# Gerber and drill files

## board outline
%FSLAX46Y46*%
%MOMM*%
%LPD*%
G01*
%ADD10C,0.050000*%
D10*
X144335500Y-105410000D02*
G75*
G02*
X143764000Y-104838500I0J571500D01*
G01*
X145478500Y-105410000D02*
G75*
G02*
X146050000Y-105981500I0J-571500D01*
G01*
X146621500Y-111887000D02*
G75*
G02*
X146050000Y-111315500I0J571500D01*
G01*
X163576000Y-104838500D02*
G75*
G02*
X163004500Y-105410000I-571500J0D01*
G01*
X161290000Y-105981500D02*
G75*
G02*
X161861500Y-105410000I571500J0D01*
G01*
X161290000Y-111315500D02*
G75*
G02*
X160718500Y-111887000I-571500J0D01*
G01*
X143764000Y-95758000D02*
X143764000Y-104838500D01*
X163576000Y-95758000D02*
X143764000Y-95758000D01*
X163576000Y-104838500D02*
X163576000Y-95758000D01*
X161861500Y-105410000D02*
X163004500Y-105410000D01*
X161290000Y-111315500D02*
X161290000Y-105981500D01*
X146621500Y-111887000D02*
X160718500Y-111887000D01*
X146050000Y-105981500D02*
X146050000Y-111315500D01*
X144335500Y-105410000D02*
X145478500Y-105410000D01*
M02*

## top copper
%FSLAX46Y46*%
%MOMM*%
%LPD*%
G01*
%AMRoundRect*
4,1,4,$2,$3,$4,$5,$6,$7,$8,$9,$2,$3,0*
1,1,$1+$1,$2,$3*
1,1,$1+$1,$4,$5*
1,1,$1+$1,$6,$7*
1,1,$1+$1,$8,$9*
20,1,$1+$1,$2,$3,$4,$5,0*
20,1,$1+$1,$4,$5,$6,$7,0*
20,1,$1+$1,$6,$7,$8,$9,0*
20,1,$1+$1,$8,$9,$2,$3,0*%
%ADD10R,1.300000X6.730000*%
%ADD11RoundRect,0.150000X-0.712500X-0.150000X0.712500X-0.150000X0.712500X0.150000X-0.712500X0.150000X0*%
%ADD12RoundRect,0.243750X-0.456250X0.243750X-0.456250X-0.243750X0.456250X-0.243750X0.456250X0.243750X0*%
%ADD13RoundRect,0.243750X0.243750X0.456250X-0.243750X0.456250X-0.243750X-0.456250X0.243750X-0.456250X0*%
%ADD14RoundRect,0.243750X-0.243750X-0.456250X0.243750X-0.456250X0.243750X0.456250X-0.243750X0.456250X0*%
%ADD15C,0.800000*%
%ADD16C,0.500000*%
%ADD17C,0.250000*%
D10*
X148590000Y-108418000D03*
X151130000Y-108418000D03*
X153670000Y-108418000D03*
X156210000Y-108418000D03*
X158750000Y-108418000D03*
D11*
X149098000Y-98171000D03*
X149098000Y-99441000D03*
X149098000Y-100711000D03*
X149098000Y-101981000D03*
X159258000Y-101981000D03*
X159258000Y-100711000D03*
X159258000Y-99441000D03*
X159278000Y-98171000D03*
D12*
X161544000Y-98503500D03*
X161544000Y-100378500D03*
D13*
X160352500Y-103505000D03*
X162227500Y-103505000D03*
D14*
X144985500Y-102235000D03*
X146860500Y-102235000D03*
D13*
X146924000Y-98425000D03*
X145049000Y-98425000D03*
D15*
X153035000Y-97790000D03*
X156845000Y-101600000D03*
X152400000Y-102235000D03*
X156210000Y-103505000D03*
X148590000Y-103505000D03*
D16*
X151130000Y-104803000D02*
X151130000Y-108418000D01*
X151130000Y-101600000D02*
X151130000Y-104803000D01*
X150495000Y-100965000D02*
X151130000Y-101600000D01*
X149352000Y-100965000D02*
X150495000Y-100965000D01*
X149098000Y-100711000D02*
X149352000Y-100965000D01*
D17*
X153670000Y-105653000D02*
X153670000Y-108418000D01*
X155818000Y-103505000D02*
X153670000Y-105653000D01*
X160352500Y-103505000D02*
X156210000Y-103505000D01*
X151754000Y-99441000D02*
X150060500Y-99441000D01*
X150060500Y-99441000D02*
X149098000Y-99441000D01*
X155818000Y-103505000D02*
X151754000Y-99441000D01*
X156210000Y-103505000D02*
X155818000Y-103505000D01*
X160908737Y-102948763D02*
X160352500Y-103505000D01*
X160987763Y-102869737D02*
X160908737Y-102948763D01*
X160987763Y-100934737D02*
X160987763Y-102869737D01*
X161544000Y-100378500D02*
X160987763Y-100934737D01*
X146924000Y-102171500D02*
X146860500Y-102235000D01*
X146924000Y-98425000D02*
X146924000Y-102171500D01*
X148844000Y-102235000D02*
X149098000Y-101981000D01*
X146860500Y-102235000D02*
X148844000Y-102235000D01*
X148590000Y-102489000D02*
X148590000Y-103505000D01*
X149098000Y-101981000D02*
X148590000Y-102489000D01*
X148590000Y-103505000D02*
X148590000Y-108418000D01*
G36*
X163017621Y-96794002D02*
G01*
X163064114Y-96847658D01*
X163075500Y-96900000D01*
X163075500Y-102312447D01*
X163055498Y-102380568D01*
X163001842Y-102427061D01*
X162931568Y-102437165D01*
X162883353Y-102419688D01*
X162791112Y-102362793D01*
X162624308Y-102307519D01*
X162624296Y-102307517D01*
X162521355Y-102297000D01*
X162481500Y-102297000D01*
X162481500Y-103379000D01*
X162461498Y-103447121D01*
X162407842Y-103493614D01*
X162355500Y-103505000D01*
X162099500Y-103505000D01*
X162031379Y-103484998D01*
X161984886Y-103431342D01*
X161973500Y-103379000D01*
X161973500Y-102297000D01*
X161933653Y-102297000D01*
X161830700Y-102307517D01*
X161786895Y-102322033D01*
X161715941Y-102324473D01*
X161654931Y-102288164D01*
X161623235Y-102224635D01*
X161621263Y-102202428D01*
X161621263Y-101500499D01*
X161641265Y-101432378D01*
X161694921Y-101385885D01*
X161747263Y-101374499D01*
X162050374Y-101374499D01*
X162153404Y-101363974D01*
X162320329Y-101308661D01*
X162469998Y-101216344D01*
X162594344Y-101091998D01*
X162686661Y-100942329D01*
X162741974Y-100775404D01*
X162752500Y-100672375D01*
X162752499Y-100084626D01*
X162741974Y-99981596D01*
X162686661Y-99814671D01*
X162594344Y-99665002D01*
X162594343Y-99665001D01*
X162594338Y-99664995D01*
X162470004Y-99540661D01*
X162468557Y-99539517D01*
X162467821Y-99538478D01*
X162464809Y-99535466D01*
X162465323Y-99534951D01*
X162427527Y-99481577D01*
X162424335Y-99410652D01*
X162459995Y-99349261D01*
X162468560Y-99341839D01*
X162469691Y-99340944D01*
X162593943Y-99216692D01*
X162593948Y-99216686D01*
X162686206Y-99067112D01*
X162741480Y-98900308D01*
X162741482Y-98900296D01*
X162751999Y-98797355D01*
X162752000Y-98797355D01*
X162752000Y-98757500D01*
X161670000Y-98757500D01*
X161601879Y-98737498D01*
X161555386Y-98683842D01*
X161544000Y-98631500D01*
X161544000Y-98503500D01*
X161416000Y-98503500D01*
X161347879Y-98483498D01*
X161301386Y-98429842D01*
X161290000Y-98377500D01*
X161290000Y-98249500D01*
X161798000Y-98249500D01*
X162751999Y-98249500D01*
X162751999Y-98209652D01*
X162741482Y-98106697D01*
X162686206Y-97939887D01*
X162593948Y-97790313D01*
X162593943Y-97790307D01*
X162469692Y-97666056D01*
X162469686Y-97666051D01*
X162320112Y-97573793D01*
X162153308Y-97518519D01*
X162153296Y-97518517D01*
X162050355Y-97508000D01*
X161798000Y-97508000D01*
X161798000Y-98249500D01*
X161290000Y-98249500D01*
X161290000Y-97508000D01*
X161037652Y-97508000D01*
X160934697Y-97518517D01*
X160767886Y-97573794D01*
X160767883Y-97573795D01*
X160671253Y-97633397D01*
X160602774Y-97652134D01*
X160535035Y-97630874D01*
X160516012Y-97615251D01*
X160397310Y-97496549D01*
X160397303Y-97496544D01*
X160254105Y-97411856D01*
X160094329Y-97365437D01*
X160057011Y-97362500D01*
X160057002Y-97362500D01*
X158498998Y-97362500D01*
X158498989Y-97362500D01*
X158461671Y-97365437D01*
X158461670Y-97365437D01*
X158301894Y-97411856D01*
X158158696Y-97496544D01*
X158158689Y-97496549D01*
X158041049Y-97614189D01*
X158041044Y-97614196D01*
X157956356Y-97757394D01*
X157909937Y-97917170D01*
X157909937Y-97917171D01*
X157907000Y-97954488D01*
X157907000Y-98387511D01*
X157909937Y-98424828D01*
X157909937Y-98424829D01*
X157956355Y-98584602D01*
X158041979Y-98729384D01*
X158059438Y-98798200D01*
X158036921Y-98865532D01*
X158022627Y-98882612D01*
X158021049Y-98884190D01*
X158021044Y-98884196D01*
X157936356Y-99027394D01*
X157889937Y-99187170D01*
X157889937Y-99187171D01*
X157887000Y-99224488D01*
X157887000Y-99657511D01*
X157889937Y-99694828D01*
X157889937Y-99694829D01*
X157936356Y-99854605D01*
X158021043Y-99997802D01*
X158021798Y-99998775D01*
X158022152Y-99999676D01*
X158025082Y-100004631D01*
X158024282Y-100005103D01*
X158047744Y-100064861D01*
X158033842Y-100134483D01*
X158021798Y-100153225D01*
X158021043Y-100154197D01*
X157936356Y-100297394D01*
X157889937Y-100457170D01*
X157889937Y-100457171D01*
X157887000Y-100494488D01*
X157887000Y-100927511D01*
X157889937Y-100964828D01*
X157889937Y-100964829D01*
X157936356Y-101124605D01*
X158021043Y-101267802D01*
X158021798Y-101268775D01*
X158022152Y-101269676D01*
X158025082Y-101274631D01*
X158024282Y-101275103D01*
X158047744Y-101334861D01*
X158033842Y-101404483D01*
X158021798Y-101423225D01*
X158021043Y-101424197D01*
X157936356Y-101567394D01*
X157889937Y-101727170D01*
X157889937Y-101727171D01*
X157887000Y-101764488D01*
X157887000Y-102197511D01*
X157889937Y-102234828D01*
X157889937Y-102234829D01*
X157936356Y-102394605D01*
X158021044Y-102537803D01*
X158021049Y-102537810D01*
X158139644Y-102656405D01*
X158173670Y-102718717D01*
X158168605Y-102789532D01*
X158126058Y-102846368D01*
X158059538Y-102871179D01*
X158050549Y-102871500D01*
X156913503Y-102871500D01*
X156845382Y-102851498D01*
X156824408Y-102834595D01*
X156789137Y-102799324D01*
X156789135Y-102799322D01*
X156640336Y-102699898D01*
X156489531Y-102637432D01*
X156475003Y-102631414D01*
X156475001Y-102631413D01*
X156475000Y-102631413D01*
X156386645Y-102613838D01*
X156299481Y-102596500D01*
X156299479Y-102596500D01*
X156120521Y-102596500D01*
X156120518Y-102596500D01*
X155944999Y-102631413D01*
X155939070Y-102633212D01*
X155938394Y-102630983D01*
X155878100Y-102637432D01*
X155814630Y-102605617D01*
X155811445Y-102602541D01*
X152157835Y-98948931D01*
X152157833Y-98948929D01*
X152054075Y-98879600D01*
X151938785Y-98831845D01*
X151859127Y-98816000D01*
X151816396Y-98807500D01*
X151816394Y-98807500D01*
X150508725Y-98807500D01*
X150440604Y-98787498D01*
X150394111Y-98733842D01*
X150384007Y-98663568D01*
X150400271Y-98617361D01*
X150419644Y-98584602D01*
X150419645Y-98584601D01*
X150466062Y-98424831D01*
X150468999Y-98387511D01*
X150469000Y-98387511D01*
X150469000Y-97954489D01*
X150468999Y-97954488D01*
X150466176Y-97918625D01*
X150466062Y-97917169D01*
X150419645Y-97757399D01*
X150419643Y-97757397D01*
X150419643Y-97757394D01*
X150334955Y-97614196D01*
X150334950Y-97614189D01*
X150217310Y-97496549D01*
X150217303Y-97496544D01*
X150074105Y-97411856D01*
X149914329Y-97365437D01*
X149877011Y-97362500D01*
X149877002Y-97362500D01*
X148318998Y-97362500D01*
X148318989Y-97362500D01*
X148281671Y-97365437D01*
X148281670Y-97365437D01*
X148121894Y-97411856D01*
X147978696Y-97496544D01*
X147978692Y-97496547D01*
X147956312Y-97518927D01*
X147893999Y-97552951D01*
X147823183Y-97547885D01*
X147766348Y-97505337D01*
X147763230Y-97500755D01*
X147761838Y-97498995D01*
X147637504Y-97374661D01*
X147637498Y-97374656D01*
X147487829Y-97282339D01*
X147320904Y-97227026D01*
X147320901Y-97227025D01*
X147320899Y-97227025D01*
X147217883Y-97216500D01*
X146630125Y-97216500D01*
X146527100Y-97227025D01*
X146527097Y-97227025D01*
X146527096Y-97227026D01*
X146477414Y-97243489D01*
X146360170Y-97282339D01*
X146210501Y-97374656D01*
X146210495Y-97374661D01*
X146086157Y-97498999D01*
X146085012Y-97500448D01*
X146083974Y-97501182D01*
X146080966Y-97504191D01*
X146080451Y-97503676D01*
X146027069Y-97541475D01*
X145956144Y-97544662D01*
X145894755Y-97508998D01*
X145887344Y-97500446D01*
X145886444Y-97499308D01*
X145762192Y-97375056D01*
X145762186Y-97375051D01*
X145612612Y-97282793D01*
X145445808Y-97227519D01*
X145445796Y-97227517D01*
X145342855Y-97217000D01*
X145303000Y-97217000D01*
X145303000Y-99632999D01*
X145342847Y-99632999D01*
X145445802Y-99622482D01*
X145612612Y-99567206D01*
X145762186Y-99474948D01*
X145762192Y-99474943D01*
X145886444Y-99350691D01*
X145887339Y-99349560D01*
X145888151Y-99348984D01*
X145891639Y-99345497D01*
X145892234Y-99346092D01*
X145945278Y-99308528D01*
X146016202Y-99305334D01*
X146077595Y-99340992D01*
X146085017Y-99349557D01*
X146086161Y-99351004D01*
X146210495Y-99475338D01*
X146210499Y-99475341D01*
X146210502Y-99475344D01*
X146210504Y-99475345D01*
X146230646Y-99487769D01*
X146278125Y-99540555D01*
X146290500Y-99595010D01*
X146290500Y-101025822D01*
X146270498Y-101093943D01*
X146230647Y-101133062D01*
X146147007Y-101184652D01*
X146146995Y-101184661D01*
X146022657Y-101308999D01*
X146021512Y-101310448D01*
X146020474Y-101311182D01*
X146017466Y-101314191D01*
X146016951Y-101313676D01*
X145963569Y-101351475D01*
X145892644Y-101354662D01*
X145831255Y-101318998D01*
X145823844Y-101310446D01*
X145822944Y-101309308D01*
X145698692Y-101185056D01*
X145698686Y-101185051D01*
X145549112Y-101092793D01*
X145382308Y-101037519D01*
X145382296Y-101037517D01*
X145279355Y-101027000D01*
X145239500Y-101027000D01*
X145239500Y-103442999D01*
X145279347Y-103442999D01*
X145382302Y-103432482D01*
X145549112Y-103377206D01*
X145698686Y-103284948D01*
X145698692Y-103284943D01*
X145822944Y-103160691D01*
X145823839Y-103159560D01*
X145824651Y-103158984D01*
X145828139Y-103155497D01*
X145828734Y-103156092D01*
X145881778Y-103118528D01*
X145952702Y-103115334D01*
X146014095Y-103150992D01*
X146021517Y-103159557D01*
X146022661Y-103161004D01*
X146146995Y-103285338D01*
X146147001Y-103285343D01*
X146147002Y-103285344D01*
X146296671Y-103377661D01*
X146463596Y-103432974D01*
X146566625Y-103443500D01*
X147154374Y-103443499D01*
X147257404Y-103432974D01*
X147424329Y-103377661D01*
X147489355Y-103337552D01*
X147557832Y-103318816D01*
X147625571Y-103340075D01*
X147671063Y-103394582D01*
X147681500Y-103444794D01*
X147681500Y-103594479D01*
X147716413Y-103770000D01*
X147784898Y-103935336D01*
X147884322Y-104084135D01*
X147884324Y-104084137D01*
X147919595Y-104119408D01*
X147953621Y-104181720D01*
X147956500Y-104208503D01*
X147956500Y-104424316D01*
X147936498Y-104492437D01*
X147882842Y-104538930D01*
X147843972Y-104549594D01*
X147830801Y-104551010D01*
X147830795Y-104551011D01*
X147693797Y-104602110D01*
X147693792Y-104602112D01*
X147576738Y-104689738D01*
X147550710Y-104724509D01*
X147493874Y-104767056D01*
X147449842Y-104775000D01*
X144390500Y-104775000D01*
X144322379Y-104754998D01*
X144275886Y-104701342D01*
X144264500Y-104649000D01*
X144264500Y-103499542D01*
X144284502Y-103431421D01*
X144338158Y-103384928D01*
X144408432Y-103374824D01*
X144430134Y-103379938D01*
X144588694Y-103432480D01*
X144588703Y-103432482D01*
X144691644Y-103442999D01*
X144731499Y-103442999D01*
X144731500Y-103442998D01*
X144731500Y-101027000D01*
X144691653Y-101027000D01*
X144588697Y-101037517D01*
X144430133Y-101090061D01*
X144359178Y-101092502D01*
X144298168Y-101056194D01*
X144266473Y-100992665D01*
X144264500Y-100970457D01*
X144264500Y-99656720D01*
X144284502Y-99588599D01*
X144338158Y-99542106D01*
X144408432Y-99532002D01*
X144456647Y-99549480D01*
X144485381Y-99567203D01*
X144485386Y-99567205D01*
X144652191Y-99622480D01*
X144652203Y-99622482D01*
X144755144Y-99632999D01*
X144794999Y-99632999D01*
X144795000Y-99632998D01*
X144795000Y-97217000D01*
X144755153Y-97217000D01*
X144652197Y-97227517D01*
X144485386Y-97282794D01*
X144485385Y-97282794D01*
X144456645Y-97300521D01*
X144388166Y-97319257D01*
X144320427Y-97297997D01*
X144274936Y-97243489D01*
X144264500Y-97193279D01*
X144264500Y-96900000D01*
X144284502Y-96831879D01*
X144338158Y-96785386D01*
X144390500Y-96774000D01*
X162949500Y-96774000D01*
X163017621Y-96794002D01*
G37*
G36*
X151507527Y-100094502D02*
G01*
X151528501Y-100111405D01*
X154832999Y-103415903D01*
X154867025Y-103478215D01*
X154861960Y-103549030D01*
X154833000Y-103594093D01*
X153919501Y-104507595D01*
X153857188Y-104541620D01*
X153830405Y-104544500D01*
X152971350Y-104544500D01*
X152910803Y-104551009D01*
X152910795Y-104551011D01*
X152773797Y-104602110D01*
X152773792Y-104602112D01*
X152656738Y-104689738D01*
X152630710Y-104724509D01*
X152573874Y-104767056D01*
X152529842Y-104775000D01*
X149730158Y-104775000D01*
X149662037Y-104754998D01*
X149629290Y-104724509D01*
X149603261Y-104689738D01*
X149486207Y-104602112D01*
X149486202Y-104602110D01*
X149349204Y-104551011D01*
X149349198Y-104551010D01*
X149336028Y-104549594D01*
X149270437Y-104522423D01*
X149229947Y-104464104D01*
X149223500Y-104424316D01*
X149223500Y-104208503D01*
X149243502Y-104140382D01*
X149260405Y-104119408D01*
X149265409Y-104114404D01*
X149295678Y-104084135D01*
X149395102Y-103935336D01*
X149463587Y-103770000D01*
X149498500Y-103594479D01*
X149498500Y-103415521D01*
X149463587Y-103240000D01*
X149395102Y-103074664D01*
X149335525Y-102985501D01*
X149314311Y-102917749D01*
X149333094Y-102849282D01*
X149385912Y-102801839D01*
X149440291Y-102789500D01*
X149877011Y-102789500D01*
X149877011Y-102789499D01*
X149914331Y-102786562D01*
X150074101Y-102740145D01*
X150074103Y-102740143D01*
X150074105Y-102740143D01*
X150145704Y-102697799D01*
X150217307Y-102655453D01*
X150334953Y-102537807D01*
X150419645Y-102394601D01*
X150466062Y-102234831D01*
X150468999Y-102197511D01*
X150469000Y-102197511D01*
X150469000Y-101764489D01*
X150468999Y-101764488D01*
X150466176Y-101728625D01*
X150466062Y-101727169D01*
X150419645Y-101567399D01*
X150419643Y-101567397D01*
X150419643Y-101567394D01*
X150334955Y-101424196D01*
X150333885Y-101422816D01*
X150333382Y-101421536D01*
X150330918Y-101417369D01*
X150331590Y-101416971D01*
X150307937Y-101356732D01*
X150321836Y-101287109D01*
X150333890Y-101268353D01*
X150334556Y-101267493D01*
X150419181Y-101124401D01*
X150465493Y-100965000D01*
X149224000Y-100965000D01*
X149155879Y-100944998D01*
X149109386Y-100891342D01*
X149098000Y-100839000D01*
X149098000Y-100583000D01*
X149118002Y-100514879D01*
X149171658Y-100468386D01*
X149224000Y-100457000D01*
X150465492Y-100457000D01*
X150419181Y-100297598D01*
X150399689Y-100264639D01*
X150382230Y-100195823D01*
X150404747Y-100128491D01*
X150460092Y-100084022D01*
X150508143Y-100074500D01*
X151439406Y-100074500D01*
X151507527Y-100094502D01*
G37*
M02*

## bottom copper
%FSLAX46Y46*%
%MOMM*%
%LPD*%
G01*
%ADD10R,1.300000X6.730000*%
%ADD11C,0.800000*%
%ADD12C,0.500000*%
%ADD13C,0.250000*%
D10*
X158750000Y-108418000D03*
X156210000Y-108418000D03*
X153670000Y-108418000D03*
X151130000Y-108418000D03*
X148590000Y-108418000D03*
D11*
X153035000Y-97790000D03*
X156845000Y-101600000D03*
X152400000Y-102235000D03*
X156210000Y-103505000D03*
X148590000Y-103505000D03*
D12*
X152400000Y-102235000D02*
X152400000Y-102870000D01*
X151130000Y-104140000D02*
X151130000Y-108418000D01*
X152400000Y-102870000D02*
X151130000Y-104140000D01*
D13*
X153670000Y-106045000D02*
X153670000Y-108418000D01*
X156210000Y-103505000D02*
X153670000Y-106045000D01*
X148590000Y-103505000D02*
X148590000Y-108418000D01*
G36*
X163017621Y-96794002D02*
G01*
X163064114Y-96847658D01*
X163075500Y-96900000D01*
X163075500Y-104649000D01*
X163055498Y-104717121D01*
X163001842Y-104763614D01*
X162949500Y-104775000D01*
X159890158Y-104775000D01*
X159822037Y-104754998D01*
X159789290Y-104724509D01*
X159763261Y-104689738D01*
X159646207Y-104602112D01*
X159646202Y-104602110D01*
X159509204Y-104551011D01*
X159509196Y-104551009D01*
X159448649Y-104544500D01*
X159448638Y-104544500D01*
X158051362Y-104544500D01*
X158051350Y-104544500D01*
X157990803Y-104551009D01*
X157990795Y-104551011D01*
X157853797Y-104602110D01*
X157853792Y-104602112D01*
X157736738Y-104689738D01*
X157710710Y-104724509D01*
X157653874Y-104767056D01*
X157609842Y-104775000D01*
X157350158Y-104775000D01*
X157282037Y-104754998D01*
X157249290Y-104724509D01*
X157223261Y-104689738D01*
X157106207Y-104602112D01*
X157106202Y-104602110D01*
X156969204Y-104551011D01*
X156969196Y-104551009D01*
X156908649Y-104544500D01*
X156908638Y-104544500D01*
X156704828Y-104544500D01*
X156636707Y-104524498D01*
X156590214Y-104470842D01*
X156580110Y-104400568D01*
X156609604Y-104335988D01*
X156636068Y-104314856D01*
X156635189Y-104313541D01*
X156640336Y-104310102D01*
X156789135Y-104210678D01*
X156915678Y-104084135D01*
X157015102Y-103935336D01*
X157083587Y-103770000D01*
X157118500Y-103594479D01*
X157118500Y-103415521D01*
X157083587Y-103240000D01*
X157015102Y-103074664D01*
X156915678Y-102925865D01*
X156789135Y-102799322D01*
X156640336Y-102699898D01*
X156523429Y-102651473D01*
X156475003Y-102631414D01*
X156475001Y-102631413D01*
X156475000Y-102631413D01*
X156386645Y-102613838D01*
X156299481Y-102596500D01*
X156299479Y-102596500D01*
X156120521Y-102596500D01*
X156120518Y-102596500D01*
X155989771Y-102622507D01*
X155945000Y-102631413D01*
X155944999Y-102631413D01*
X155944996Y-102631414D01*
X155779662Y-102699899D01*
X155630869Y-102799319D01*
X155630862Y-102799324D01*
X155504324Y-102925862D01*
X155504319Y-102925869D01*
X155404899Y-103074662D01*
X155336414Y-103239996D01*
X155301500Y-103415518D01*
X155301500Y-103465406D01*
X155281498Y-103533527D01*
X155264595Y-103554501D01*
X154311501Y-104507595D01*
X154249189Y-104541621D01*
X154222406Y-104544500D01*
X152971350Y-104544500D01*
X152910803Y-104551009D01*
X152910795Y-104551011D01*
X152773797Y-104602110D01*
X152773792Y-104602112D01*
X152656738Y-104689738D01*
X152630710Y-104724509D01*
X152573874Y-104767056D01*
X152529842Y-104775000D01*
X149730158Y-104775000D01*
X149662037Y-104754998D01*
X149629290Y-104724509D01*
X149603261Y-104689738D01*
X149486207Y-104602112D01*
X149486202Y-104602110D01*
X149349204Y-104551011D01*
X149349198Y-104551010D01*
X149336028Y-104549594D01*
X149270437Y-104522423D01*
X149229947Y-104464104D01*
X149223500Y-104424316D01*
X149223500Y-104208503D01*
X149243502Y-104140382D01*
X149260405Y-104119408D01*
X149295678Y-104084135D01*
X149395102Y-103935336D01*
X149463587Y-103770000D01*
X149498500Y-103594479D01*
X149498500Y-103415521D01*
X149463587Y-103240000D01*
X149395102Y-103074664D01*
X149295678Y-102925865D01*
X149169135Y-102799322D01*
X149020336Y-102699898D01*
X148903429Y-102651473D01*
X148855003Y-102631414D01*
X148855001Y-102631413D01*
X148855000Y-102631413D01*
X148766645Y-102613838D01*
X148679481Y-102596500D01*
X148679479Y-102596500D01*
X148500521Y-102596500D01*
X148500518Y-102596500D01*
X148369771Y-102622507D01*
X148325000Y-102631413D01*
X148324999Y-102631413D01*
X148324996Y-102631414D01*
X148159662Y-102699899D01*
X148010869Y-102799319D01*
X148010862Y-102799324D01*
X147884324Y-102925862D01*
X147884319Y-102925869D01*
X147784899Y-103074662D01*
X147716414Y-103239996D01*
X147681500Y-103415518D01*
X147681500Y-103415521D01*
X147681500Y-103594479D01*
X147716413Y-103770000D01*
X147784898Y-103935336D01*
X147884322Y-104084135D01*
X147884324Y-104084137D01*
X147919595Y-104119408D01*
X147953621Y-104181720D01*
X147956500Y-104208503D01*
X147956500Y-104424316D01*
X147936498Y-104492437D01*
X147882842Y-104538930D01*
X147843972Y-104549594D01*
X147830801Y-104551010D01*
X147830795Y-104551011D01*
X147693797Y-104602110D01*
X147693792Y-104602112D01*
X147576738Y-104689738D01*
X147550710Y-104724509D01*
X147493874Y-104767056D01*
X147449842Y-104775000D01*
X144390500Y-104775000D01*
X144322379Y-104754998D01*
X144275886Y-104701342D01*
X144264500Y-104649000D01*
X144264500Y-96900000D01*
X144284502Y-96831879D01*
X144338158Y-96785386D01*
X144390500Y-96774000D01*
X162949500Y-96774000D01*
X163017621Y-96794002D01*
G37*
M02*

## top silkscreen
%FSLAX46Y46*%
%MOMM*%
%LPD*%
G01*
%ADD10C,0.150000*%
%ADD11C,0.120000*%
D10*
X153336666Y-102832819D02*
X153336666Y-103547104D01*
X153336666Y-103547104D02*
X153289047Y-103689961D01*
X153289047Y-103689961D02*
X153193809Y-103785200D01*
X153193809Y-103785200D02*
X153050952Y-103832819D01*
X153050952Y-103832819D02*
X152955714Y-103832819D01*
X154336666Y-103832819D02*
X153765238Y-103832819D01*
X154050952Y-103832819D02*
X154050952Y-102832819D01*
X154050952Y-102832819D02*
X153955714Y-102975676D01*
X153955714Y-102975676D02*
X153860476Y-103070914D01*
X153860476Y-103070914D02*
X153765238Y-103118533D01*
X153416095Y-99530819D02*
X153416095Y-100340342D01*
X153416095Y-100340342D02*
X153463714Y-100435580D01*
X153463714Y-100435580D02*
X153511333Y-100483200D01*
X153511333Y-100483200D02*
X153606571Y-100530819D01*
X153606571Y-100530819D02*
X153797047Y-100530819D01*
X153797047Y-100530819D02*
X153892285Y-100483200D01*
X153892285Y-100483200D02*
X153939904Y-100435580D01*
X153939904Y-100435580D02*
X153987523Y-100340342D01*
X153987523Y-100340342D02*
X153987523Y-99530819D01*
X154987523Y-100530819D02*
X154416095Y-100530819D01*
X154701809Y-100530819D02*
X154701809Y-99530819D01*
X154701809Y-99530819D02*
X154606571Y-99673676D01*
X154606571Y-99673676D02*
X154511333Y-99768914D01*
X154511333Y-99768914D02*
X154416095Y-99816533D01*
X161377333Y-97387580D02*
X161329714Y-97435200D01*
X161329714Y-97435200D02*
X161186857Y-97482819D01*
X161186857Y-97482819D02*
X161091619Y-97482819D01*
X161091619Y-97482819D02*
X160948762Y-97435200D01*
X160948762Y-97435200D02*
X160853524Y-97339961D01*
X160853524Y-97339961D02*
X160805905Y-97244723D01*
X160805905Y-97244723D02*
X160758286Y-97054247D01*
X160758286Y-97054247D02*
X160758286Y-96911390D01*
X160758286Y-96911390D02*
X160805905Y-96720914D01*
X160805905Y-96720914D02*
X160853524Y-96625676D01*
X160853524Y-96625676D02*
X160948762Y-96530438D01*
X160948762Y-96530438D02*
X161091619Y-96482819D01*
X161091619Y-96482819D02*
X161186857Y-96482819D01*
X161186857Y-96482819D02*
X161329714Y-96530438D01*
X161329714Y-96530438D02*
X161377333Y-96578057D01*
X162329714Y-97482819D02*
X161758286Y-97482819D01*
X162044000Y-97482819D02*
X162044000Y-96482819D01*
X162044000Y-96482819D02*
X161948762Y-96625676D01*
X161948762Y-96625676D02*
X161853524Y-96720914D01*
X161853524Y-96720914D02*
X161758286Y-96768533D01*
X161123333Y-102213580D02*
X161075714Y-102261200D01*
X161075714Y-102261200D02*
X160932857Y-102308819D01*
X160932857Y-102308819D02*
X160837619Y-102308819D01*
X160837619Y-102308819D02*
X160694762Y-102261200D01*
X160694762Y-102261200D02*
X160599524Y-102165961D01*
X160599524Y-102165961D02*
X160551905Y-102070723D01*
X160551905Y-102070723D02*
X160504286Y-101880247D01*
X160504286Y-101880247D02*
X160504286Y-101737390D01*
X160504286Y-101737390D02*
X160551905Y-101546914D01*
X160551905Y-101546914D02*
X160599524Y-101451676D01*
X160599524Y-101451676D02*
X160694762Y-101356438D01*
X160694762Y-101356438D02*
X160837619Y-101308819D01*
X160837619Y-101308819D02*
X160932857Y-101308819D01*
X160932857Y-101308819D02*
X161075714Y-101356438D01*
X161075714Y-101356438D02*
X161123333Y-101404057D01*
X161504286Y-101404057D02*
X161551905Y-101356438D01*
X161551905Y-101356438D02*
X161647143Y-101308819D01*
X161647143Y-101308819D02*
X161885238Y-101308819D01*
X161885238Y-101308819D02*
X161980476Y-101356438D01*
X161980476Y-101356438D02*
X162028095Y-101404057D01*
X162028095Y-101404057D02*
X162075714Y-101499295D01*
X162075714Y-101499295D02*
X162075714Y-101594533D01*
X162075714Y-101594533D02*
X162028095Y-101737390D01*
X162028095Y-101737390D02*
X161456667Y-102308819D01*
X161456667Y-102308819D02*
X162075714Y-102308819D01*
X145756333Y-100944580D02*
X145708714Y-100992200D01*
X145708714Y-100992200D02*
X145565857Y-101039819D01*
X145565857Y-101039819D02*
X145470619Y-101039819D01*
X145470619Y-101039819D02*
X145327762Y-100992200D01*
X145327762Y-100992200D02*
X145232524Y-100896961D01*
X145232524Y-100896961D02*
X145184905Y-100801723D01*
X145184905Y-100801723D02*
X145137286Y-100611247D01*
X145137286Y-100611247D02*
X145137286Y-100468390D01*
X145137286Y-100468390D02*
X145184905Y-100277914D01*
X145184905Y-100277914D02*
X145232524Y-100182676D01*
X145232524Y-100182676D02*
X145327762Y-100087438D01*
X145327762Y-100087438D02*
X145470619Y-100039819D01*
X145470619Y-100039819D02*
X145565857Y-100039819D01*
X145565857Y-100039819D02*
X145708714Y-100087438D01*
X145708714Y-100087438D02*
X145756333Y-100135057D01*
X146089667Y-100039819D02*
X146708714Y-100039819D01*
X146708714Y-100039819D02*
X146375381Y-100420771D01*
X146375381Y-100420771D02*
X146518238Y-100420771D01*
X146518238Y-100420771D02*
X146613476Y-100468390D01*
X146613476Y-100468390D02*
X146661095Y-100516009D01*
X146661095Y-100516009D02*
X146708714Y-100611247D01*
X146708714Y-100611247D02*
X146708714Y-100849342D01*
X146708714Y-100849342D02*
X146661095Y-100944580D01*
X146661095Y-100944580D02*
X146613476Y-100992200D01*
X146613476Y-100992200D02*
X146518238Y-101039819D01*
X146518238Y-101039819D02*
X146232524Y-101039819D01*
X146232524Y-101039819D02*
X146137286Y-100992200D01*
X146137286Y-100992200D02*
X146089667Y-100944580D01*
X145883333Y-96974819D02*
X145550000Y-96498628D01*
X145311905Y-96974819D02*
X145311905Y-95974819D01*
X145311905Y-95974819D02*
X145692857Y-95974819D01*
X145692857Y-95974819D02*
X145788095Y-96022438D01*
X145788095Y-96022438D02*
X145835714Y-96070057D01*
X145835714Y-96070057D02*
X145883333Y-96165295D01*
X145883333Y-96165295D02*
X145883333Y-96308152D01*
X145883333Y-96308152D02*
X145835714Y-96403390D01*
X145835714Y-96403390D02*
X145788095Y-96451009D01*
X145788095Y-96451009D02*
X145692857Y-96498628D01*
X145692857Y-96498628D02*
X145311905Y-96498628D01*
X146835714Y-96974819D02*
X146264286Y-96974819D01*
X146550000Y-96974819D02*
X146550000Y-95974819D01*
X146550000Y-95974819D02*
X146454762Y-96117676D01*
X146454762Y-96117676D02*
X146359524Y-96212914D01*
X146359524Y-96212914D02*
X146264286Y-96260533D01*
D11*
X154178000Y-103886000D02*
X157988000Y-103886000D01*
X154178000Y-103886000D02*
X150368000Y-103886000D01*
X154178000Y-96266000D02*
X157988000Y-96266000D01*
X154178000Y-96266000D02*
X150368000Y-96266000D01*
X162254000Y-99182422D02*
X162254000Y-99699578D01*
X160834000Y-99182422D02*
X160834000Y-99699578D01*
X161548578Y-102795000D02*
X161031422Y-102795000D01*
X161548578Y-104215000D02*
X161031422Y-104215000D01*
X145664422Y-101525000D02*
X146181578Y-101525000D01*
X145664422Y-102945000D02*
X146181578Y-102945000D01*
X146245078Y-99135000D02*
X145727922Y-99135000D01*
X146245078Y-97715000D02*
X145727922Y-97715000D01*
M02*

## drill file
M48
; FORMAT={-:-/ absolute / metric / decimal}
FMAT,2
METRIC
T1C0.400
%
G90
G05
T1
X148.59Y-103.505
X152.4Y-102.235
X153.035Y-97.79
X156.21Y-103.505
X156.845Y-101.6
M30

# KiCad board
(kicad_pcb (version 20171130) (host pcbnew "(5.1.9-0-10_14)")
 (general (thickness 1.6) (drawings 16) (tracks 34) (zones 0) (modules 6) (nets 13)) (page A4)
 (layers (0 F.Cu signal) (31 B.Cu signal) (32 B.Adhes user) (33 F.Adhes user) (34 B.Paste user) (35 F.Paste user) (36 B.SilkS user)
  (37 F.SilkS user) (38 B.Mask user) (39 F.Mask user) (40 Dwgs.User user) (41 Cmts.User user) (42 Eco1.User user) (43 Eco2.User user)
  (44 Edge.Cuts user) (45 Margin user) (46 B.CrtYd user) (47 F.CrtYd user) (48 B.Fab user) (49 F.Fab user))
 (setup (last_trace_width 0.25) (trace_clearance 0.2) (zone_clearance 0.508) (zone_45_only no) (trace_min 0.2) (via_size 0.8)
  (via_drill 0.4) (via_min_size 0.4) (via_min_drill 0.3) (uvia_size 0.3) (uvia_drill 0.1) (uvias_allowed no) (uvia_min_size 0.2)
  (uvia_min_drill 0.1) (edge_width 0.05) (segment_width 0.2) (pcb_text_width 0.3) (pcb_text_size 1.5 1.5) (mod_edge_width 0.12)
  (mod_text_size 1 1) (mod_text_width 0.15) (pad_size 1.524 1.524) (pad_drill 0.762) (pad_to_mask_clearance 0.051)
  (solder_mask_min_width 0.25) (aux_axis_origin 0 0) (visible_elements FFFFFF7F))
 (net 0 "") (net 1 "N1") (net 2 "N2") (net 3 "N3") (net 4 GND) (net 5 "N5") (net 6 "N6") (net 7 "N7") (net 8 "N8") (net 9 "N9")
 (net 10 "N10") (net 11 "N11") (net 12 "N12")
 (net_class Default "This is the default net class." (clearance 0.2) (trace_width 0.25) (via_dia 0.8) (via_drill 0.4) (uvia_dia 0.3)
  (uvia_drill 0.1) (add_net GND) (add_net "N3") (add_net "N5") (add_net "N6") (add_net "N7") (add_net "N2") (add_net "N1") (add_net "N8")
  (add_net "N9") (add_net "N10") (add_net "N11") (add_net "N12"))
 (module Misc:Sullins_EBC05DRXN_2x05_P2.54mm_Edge (layer F.Cu) (at 148.59 105.918)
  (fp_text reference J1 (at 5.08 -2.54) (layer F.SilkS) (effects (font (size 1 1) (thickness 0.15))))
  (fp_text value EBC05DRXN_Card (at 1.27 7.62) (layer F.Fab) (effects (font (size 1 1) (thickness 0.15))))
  (pad B5 connect rect (at 10.16 2.5) (size 1.3 6.73) (layers B.Cu) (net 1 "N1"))
  (pad B4 connect rect (at 7.62 2.5) (size 1.3 6.73) (layers B.Cu) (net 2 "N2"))
  (pad B3 connect rect (at 5.08 2.5) (size 1.3 6.73) (layers B.Cu) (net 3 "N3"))
  (pad B2 connect rect (at 2.54 2.5) (size 1.3 6.73) (layers B.Cu) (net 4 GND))
  (pad B1 connect rect (at 0 2.5) (size 1.3 6.73) (layers B.Cu) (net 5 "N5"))
  (pad A1 connect rect (at 0 2.5) (size 1.3 6.73) (layers F.Cu) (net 5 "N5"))
  (pad A2 connect rect (at 2.54 2.5) (size 1.3 6.73) (layers F.Cu) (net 4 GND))
  (pad A3 connect rect (at 5.08 2.5) (size 1.3 6.73) (layers F.Cu) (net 3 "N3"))
  (pad A4 connect rect (at 7.62 2.5) (size 1.3 6.73) (layers F.Cu) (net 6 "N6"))
  (pad A5 connect rect (at 10.16 2.5) (size 1.3 6.73) (layers F.Cu) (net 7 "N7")))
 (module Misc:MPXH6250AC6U (layer F.Cu) (at 154.178 100.076)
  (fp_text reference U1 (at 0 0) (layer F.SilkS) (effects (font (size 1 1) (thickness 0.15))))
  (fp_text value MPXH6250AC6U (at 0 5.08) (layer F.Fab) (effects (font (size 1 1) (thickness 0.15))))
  (fp_line (start 0 3.81) (end 3.81 3.81) (layer F.SilkS) (width 0.12))
  (fp_line (start 0 3.81) (end -3.81 3.81) (layer F.SilkS) (width 0.12))
  (fp_line (start 0 -3.81) (end 3.81 -3.81) (layer F.SilkS) (width 0.12))
  (fp_line (start 0 -3.81) (end -3.81 -3.81) (layer F.SilkS) (width 0.12))
  (pad 1 smd roundrect (at -5.08 -1.905) (size 1.725 0.6) (layers F.Cu F.Paste F.Mask) (roundrect_rratio 0.25) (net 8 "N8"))
  (pad 2 smd roundrect (at -5.08 -0.635) (size 1.725 0.6) (layers F.Cu F.Paste F.Mask) (roundrect_rratio 0.25) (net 3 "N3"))
  (pad 3 smd roundrect (at -5.08 0.635) (size 1.725 0.6) (layers F.Cu F.Paste F.Mask) (roundrect_rratio 0.25) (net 4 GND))
  (pad 4 smd roundrect (at -5.08 1.905) (size 1.725 0.6) (layers F.Cu F.Paste F.Mask) (roundrect_rratio 0.25) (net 5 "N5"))
  (pad 5 smd roundrect (at 5.08 1.905) (size 1.725 0.6) (layers F.Cu F.Paste F.Mask) (roundrect_rratio 0.25) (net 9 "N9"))
  (pad 6 smd roundrect (at 5.08 0.635) (size 1.725 0.6) (layers F.Cu F.Paste F.Mask) (roundrect_rratio 0.25) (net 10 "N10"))
  (pad 7 smd roundrect (at 5.08 -0.635) (size 1.725 0.6) (layers F.Cu F.Paste F.Mask) (roundrect_rratio 0.25) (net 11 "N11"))
  (pad 8 smd roundrect (at 5.1 -1.905) (size 1.725 0.6) (layers F.Cu F.Paste F.Mask) (roundrect_rratio 0.25) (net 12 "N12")))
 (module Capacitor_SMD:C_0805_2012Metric (layer F.Cu) (at 161.544 99.441 270)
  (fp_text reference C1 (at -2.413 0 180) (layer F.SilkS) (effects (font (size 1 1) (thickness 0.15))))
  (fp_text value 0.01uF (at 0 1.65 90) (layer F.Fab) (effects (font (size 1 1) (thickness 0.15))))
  (fp_line (start -0.258578 -0.71) (end 0.258578 -0.71) (layer F.SilkS) (width 0.12))
  (fp_line (start -0.258578 0.71) (end 0.258578 0.71) (layer F.SilkS) (width 0.12))
  (pad 1 smd roundrect (at -0.9375 0 270) (size 0.975 1.4) (layers F.Cu F.Paste F.Mask) (roundrect_rratio 0.25) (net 4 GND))
  (pad 2 smd roundrect (at 0.9375 0 270) (size 0.975 1.4) (layers F.Cu F.Paste F.Mask) (roundrect_rratio 0.25) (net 3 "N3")))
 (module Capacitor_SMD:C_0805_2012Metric (layer F.Cu) (at 161.29 103.505 180)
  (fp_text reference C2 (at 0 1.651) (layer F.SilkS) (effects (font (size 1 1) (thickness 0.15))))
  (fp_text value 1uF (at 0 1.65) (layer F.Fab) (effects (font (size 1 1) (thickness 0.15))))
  (fp_line (start -0.258578 0.71) (end 0.258578 0.71) (layer F.SilkS) (width 0.12))
  (fp_line (start -0.258578 -0.71) (end 0.258578 -0.71) (layer F.SilkS) (width 0.12))
  (pad 2 smd roundrect (at 0.9375 0 180) (size 0.975 1.4) (layers F.Cu F.Paste F.Mask) (roundrect_rratio 0.25) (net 3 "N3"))
  (pad 1 smd roundrect (at -0.9375 0 180) (size 0.975 1.4) (layers F.Cu F.Paste F.Mask) (roundrect_rratio 0.25) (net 4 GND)))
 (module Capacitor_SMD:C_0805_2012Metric (layer F.Cu) (at 145.923 102.235)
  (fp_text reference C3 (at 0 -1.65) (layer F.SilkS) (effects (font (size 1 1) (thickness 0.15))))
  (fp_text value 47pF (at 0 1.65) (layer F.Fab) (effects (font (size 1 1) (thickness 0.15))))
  (fp_line (start -0.258578 -0.71) (end 0.258578 -0.71) (layer F.SilkS) (width 0.12))
  (fp_line (start -0.258578 0.71) (end 0.258578 0.71) (layer F.SilkS) (width 0.12))
  (pad 1 smd roundrect (at -0.9375 0) (size 0.975 1.4) (layers F.Cu F.Paste F.Mask) (roundrect_rratio 0.25) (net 4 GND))
  (pad 2 smd roundrect (at 0.9375 0) (size 0.975 1.4) (layers F.Cu F.Paste F.Mask) (roundrect_rratio 0.25) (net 5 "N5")))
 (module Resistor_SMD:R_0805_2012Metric (layer F.Cu) (at 145.9865 98.425 180)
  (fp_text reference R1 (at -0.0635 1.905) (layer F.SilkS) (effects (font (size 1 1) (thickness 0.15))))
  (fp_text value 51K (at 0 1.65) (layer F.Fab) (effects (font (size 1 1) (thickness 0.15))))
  (fp_line (start -0.258578 -0.71) (end 0.258578 -0.71) (layer F.SilkS) (width 0.12))
  (fp_line (start -0.258578 0.71) (end 0.258578 0.71) (layer F.SilkS) (width 0.12))
  (pad 1 smd roundrect (at -0.9375 0 180) (size 0.975 1.4) (layers F.Cu F.Paste F.Mask) (roundrect_rratio 0.25) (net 5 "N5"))
  (pad 2 smd roundrect (at 0.9375 0 180) (size 0.975 1.4) (layers F.Cu F.Paste F.Mask) (roundrect_rratio 0.25) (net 4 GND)))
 (gr_arc (start 144.3355 104.8385) (end 143.764 104.8385) (angle -90) (layer Edge.Cuts) (width 0.05))
 (gr_arc (start 145.4785 105.9815) (end 146.05 105.9815) (angle -90) (layer Edge.Cuts) (width 0.05))
 (gr_arc (start 146.6215 111.3155) (end 146.05 111.3155) (angle -90) (layer Edge.Cuts) (width 0.05))
 (gr_arc (start 163.0045 104.8385) (end 163.0045 105.41) (angle -90) (layer Edge.Cuts) (width 0.05))
 (gr_arc (start 161.8615 105.9815) (end 161.8615 105.41) (angle -90) (layer Edge.Cuts) (width 0.05))
 (gr_arc (start 160.7185 111.3155) (end 160.7185 111.887) (angle -90) (layer Edge.Cuts) (width 0.05))
 (gr_line (start 143.764 95.758) (end 143.764 104.8385) (layer Edge.Cuts) (width 0.05))
 (gr_line (start 163.576 95.758) (end 143.764 95.758) (layer Edge.Cuts) (width 0.05))
 (gr_line (start 163.576 104.8385) (end 163.576 95.758) (layer Edge.Cuts) (width 0.05))
 (gr_line (start 161.8615 105.41) (end 163.0045 105.41) (layer Edge.Cuts) (width 0.05))
 (gr_line (start 161.29 111.3155) (end 161.29 105.9815) (layer Edge.Cuts) (width 0.05))
 (gr_line (start 146.6215 111.887) (end 160.7185 111.887) (layer Edge.Cuts) (width 0.05))
 (gr_line (start 146.05 105.9815) (end 146.05 111.3155) (layer Edge.Cuts) (width 0.05))
 (gr_line (start 144.3355 105.41) (end 145.4785 105.41) (layer Edge.Cuts) (width 0.05))
 (segment (start 151.13 104.803) (end 151.13 108.418) (width 0.5) (layer F.Cu) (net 4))
 (segment (start 151.13 101.6) (end 151.13 104.803) (width 0.5) (layer F.Cu) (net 4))
 (segment (start 150.495 100.965) (end 151.13 101.6) (width 0.5) (layer F.Cu) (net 4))
 (segment (start 149.352 100.965) (end 150.495 100.965) (width 0.5) (layer F.Cu) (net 4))
 (segment (start 149.098 100.711) (end 149.352 100.965) (width 0.5) (layer F.Cu) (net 4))
 (via (at 153.035 97.79) (size 0.8) (drill 0.4) (layers F.Cu B.Cu) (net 4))
 (via (at 156.845 101.6) (size 0.8) (drill 0.4) (layers F.Cu B.Cu) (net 4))
 (via (at 152.4 102.235) (size 0.8) (drill 0.4) (layers F.Cu B.Cu) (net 4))
 (segment (start 152.4 102.235) (end 152.4 102.87) (width 0.5) (layer B.Cu) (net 4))
 (segment (start 151.13 104.14) (end 151.13 108.418) (width 0.5) (layer B.Cu) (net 4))
 (segment (start 152.4 102.87) (end 151.13 104.14) (width 0.5) (layer B.Cu) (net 4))
 (segment (start 153.67 105.653) (end 153.67 108.418) (width 0.25) (layer F.Cu) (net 3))
 (segment (start 155.818 103.505) (end 153.67 105.653) (width 0.25) (layer F.Cu) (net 3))
 (segment (start 160.3525 103.505) (end 156.21 103.505) (width 0.25) (layer F.Cu) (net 3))
 (segment (start 151.754 99.441) (end 150.0605 99.441) (width 0.25) (layer F.Cu) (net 3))
 (segment (start 150.0605 99.441) (end 149.098 99.441) (width 0.25) (layer F.Cu) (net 3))
 (segment (start 155.818 103.505) (end 151.754 99.441) (width 0.25) (layer F.Cu) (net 3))
 (segment (start 156.21 103.505) (end 155.818 103.505) (width 0.25) (layer F.Cu) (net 3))
 (via (at 156.21 103.505) (size 0.8) (drill 0.4) (layers F.Cu B.Cu) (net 3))
 (segment (start 153.67 106.045) (end 153.67 108.418) (width 0.25) (layer B.Cu) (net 3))
 (segment (start 156.21 103.505) (end 153.67 106.045) (width 0.25) (layer B.Cu) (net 3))
 (segment (start 160.908737 102.948763) (end 160.3525 103.505) (width 0.25) (layer F.Cu) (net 3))
 (segment (start 160.987763 102.869737) (end 160.908737 102.948763) (width 0.25) (layer F.Cu) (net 3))
 (segment (start 160.987763 100.934737) (end 160.987763 102.869737) (width 0.25) (layer F.Cu) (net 3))
 (segment (start 161.544 100.3785) (end 160.987763 100.934737) (width 0.25) (layer F.Cu) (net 3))
 (segment (start 146.924 102.1715) (end 146.8605 102.235) (width 0.25) (layer F.Cu) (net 5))
 (segment (start 146.924 98.425) (end 146.924 102.1715) (width 0.25) (layer F.Cu) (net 5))
 (segment (start 148.844 102.235) (end 149.098 101.981) (width 0.25) (layer F.Cu) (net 5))
 (segment (start 146.8605 102.235) (end 148.844 102.235) (width 0.25) (layer F.Cu) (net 5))
 (segment (start 148.59 102.489) (end 148.59 103.505) (width 0.25) (layer F.Cu) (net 5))
 (segment (start 149.098 101.981) (end 148.59 102.489) (width 0.25) (layer F.Cu) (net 5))
 (segment (start 148.59 103.505) (end 148.59 108.418) (width 0.25) (layer F.Cu) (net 5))
 (via (at 148.59 103.505) (size 0.8) (drill 0.4) (layers F.Cu B.Cu) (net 5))
 (segment (start 148.59 103.505) (end 148.59 108.418) (width 0.25) (layer B.Cu) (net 5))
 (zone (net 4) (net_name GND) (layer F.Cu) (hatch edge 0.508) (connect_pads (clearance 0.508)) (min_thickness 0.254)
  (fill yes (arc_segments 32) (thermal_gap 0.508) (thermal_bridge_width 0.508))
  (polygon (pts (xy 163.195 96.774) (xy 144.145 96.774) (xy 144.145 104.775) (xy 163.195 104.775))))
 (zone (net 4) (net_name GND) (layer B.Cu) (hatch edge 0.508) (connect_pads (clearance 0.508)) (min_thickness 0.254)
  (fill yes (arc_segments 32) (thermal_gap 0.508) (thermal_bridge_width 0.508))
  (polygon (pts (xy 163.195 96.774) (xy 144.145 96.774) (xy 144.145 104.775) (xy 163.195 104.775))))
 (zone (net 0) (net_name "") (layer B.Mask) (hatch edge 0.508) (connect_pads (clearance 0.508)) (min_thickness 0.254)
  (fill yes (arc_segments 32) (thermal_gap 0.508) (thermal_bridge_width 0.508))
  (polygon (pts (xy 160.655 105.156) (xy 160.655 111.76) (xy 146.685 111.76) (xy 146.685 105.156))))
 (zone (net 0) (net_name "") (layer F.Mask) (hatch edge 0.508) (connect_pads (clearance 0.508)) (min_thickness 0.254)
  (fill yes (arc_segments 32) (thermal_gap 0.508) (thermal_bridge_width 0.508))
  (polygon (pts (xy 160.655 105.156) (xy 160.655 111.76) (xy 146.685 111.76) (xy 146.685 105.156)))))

